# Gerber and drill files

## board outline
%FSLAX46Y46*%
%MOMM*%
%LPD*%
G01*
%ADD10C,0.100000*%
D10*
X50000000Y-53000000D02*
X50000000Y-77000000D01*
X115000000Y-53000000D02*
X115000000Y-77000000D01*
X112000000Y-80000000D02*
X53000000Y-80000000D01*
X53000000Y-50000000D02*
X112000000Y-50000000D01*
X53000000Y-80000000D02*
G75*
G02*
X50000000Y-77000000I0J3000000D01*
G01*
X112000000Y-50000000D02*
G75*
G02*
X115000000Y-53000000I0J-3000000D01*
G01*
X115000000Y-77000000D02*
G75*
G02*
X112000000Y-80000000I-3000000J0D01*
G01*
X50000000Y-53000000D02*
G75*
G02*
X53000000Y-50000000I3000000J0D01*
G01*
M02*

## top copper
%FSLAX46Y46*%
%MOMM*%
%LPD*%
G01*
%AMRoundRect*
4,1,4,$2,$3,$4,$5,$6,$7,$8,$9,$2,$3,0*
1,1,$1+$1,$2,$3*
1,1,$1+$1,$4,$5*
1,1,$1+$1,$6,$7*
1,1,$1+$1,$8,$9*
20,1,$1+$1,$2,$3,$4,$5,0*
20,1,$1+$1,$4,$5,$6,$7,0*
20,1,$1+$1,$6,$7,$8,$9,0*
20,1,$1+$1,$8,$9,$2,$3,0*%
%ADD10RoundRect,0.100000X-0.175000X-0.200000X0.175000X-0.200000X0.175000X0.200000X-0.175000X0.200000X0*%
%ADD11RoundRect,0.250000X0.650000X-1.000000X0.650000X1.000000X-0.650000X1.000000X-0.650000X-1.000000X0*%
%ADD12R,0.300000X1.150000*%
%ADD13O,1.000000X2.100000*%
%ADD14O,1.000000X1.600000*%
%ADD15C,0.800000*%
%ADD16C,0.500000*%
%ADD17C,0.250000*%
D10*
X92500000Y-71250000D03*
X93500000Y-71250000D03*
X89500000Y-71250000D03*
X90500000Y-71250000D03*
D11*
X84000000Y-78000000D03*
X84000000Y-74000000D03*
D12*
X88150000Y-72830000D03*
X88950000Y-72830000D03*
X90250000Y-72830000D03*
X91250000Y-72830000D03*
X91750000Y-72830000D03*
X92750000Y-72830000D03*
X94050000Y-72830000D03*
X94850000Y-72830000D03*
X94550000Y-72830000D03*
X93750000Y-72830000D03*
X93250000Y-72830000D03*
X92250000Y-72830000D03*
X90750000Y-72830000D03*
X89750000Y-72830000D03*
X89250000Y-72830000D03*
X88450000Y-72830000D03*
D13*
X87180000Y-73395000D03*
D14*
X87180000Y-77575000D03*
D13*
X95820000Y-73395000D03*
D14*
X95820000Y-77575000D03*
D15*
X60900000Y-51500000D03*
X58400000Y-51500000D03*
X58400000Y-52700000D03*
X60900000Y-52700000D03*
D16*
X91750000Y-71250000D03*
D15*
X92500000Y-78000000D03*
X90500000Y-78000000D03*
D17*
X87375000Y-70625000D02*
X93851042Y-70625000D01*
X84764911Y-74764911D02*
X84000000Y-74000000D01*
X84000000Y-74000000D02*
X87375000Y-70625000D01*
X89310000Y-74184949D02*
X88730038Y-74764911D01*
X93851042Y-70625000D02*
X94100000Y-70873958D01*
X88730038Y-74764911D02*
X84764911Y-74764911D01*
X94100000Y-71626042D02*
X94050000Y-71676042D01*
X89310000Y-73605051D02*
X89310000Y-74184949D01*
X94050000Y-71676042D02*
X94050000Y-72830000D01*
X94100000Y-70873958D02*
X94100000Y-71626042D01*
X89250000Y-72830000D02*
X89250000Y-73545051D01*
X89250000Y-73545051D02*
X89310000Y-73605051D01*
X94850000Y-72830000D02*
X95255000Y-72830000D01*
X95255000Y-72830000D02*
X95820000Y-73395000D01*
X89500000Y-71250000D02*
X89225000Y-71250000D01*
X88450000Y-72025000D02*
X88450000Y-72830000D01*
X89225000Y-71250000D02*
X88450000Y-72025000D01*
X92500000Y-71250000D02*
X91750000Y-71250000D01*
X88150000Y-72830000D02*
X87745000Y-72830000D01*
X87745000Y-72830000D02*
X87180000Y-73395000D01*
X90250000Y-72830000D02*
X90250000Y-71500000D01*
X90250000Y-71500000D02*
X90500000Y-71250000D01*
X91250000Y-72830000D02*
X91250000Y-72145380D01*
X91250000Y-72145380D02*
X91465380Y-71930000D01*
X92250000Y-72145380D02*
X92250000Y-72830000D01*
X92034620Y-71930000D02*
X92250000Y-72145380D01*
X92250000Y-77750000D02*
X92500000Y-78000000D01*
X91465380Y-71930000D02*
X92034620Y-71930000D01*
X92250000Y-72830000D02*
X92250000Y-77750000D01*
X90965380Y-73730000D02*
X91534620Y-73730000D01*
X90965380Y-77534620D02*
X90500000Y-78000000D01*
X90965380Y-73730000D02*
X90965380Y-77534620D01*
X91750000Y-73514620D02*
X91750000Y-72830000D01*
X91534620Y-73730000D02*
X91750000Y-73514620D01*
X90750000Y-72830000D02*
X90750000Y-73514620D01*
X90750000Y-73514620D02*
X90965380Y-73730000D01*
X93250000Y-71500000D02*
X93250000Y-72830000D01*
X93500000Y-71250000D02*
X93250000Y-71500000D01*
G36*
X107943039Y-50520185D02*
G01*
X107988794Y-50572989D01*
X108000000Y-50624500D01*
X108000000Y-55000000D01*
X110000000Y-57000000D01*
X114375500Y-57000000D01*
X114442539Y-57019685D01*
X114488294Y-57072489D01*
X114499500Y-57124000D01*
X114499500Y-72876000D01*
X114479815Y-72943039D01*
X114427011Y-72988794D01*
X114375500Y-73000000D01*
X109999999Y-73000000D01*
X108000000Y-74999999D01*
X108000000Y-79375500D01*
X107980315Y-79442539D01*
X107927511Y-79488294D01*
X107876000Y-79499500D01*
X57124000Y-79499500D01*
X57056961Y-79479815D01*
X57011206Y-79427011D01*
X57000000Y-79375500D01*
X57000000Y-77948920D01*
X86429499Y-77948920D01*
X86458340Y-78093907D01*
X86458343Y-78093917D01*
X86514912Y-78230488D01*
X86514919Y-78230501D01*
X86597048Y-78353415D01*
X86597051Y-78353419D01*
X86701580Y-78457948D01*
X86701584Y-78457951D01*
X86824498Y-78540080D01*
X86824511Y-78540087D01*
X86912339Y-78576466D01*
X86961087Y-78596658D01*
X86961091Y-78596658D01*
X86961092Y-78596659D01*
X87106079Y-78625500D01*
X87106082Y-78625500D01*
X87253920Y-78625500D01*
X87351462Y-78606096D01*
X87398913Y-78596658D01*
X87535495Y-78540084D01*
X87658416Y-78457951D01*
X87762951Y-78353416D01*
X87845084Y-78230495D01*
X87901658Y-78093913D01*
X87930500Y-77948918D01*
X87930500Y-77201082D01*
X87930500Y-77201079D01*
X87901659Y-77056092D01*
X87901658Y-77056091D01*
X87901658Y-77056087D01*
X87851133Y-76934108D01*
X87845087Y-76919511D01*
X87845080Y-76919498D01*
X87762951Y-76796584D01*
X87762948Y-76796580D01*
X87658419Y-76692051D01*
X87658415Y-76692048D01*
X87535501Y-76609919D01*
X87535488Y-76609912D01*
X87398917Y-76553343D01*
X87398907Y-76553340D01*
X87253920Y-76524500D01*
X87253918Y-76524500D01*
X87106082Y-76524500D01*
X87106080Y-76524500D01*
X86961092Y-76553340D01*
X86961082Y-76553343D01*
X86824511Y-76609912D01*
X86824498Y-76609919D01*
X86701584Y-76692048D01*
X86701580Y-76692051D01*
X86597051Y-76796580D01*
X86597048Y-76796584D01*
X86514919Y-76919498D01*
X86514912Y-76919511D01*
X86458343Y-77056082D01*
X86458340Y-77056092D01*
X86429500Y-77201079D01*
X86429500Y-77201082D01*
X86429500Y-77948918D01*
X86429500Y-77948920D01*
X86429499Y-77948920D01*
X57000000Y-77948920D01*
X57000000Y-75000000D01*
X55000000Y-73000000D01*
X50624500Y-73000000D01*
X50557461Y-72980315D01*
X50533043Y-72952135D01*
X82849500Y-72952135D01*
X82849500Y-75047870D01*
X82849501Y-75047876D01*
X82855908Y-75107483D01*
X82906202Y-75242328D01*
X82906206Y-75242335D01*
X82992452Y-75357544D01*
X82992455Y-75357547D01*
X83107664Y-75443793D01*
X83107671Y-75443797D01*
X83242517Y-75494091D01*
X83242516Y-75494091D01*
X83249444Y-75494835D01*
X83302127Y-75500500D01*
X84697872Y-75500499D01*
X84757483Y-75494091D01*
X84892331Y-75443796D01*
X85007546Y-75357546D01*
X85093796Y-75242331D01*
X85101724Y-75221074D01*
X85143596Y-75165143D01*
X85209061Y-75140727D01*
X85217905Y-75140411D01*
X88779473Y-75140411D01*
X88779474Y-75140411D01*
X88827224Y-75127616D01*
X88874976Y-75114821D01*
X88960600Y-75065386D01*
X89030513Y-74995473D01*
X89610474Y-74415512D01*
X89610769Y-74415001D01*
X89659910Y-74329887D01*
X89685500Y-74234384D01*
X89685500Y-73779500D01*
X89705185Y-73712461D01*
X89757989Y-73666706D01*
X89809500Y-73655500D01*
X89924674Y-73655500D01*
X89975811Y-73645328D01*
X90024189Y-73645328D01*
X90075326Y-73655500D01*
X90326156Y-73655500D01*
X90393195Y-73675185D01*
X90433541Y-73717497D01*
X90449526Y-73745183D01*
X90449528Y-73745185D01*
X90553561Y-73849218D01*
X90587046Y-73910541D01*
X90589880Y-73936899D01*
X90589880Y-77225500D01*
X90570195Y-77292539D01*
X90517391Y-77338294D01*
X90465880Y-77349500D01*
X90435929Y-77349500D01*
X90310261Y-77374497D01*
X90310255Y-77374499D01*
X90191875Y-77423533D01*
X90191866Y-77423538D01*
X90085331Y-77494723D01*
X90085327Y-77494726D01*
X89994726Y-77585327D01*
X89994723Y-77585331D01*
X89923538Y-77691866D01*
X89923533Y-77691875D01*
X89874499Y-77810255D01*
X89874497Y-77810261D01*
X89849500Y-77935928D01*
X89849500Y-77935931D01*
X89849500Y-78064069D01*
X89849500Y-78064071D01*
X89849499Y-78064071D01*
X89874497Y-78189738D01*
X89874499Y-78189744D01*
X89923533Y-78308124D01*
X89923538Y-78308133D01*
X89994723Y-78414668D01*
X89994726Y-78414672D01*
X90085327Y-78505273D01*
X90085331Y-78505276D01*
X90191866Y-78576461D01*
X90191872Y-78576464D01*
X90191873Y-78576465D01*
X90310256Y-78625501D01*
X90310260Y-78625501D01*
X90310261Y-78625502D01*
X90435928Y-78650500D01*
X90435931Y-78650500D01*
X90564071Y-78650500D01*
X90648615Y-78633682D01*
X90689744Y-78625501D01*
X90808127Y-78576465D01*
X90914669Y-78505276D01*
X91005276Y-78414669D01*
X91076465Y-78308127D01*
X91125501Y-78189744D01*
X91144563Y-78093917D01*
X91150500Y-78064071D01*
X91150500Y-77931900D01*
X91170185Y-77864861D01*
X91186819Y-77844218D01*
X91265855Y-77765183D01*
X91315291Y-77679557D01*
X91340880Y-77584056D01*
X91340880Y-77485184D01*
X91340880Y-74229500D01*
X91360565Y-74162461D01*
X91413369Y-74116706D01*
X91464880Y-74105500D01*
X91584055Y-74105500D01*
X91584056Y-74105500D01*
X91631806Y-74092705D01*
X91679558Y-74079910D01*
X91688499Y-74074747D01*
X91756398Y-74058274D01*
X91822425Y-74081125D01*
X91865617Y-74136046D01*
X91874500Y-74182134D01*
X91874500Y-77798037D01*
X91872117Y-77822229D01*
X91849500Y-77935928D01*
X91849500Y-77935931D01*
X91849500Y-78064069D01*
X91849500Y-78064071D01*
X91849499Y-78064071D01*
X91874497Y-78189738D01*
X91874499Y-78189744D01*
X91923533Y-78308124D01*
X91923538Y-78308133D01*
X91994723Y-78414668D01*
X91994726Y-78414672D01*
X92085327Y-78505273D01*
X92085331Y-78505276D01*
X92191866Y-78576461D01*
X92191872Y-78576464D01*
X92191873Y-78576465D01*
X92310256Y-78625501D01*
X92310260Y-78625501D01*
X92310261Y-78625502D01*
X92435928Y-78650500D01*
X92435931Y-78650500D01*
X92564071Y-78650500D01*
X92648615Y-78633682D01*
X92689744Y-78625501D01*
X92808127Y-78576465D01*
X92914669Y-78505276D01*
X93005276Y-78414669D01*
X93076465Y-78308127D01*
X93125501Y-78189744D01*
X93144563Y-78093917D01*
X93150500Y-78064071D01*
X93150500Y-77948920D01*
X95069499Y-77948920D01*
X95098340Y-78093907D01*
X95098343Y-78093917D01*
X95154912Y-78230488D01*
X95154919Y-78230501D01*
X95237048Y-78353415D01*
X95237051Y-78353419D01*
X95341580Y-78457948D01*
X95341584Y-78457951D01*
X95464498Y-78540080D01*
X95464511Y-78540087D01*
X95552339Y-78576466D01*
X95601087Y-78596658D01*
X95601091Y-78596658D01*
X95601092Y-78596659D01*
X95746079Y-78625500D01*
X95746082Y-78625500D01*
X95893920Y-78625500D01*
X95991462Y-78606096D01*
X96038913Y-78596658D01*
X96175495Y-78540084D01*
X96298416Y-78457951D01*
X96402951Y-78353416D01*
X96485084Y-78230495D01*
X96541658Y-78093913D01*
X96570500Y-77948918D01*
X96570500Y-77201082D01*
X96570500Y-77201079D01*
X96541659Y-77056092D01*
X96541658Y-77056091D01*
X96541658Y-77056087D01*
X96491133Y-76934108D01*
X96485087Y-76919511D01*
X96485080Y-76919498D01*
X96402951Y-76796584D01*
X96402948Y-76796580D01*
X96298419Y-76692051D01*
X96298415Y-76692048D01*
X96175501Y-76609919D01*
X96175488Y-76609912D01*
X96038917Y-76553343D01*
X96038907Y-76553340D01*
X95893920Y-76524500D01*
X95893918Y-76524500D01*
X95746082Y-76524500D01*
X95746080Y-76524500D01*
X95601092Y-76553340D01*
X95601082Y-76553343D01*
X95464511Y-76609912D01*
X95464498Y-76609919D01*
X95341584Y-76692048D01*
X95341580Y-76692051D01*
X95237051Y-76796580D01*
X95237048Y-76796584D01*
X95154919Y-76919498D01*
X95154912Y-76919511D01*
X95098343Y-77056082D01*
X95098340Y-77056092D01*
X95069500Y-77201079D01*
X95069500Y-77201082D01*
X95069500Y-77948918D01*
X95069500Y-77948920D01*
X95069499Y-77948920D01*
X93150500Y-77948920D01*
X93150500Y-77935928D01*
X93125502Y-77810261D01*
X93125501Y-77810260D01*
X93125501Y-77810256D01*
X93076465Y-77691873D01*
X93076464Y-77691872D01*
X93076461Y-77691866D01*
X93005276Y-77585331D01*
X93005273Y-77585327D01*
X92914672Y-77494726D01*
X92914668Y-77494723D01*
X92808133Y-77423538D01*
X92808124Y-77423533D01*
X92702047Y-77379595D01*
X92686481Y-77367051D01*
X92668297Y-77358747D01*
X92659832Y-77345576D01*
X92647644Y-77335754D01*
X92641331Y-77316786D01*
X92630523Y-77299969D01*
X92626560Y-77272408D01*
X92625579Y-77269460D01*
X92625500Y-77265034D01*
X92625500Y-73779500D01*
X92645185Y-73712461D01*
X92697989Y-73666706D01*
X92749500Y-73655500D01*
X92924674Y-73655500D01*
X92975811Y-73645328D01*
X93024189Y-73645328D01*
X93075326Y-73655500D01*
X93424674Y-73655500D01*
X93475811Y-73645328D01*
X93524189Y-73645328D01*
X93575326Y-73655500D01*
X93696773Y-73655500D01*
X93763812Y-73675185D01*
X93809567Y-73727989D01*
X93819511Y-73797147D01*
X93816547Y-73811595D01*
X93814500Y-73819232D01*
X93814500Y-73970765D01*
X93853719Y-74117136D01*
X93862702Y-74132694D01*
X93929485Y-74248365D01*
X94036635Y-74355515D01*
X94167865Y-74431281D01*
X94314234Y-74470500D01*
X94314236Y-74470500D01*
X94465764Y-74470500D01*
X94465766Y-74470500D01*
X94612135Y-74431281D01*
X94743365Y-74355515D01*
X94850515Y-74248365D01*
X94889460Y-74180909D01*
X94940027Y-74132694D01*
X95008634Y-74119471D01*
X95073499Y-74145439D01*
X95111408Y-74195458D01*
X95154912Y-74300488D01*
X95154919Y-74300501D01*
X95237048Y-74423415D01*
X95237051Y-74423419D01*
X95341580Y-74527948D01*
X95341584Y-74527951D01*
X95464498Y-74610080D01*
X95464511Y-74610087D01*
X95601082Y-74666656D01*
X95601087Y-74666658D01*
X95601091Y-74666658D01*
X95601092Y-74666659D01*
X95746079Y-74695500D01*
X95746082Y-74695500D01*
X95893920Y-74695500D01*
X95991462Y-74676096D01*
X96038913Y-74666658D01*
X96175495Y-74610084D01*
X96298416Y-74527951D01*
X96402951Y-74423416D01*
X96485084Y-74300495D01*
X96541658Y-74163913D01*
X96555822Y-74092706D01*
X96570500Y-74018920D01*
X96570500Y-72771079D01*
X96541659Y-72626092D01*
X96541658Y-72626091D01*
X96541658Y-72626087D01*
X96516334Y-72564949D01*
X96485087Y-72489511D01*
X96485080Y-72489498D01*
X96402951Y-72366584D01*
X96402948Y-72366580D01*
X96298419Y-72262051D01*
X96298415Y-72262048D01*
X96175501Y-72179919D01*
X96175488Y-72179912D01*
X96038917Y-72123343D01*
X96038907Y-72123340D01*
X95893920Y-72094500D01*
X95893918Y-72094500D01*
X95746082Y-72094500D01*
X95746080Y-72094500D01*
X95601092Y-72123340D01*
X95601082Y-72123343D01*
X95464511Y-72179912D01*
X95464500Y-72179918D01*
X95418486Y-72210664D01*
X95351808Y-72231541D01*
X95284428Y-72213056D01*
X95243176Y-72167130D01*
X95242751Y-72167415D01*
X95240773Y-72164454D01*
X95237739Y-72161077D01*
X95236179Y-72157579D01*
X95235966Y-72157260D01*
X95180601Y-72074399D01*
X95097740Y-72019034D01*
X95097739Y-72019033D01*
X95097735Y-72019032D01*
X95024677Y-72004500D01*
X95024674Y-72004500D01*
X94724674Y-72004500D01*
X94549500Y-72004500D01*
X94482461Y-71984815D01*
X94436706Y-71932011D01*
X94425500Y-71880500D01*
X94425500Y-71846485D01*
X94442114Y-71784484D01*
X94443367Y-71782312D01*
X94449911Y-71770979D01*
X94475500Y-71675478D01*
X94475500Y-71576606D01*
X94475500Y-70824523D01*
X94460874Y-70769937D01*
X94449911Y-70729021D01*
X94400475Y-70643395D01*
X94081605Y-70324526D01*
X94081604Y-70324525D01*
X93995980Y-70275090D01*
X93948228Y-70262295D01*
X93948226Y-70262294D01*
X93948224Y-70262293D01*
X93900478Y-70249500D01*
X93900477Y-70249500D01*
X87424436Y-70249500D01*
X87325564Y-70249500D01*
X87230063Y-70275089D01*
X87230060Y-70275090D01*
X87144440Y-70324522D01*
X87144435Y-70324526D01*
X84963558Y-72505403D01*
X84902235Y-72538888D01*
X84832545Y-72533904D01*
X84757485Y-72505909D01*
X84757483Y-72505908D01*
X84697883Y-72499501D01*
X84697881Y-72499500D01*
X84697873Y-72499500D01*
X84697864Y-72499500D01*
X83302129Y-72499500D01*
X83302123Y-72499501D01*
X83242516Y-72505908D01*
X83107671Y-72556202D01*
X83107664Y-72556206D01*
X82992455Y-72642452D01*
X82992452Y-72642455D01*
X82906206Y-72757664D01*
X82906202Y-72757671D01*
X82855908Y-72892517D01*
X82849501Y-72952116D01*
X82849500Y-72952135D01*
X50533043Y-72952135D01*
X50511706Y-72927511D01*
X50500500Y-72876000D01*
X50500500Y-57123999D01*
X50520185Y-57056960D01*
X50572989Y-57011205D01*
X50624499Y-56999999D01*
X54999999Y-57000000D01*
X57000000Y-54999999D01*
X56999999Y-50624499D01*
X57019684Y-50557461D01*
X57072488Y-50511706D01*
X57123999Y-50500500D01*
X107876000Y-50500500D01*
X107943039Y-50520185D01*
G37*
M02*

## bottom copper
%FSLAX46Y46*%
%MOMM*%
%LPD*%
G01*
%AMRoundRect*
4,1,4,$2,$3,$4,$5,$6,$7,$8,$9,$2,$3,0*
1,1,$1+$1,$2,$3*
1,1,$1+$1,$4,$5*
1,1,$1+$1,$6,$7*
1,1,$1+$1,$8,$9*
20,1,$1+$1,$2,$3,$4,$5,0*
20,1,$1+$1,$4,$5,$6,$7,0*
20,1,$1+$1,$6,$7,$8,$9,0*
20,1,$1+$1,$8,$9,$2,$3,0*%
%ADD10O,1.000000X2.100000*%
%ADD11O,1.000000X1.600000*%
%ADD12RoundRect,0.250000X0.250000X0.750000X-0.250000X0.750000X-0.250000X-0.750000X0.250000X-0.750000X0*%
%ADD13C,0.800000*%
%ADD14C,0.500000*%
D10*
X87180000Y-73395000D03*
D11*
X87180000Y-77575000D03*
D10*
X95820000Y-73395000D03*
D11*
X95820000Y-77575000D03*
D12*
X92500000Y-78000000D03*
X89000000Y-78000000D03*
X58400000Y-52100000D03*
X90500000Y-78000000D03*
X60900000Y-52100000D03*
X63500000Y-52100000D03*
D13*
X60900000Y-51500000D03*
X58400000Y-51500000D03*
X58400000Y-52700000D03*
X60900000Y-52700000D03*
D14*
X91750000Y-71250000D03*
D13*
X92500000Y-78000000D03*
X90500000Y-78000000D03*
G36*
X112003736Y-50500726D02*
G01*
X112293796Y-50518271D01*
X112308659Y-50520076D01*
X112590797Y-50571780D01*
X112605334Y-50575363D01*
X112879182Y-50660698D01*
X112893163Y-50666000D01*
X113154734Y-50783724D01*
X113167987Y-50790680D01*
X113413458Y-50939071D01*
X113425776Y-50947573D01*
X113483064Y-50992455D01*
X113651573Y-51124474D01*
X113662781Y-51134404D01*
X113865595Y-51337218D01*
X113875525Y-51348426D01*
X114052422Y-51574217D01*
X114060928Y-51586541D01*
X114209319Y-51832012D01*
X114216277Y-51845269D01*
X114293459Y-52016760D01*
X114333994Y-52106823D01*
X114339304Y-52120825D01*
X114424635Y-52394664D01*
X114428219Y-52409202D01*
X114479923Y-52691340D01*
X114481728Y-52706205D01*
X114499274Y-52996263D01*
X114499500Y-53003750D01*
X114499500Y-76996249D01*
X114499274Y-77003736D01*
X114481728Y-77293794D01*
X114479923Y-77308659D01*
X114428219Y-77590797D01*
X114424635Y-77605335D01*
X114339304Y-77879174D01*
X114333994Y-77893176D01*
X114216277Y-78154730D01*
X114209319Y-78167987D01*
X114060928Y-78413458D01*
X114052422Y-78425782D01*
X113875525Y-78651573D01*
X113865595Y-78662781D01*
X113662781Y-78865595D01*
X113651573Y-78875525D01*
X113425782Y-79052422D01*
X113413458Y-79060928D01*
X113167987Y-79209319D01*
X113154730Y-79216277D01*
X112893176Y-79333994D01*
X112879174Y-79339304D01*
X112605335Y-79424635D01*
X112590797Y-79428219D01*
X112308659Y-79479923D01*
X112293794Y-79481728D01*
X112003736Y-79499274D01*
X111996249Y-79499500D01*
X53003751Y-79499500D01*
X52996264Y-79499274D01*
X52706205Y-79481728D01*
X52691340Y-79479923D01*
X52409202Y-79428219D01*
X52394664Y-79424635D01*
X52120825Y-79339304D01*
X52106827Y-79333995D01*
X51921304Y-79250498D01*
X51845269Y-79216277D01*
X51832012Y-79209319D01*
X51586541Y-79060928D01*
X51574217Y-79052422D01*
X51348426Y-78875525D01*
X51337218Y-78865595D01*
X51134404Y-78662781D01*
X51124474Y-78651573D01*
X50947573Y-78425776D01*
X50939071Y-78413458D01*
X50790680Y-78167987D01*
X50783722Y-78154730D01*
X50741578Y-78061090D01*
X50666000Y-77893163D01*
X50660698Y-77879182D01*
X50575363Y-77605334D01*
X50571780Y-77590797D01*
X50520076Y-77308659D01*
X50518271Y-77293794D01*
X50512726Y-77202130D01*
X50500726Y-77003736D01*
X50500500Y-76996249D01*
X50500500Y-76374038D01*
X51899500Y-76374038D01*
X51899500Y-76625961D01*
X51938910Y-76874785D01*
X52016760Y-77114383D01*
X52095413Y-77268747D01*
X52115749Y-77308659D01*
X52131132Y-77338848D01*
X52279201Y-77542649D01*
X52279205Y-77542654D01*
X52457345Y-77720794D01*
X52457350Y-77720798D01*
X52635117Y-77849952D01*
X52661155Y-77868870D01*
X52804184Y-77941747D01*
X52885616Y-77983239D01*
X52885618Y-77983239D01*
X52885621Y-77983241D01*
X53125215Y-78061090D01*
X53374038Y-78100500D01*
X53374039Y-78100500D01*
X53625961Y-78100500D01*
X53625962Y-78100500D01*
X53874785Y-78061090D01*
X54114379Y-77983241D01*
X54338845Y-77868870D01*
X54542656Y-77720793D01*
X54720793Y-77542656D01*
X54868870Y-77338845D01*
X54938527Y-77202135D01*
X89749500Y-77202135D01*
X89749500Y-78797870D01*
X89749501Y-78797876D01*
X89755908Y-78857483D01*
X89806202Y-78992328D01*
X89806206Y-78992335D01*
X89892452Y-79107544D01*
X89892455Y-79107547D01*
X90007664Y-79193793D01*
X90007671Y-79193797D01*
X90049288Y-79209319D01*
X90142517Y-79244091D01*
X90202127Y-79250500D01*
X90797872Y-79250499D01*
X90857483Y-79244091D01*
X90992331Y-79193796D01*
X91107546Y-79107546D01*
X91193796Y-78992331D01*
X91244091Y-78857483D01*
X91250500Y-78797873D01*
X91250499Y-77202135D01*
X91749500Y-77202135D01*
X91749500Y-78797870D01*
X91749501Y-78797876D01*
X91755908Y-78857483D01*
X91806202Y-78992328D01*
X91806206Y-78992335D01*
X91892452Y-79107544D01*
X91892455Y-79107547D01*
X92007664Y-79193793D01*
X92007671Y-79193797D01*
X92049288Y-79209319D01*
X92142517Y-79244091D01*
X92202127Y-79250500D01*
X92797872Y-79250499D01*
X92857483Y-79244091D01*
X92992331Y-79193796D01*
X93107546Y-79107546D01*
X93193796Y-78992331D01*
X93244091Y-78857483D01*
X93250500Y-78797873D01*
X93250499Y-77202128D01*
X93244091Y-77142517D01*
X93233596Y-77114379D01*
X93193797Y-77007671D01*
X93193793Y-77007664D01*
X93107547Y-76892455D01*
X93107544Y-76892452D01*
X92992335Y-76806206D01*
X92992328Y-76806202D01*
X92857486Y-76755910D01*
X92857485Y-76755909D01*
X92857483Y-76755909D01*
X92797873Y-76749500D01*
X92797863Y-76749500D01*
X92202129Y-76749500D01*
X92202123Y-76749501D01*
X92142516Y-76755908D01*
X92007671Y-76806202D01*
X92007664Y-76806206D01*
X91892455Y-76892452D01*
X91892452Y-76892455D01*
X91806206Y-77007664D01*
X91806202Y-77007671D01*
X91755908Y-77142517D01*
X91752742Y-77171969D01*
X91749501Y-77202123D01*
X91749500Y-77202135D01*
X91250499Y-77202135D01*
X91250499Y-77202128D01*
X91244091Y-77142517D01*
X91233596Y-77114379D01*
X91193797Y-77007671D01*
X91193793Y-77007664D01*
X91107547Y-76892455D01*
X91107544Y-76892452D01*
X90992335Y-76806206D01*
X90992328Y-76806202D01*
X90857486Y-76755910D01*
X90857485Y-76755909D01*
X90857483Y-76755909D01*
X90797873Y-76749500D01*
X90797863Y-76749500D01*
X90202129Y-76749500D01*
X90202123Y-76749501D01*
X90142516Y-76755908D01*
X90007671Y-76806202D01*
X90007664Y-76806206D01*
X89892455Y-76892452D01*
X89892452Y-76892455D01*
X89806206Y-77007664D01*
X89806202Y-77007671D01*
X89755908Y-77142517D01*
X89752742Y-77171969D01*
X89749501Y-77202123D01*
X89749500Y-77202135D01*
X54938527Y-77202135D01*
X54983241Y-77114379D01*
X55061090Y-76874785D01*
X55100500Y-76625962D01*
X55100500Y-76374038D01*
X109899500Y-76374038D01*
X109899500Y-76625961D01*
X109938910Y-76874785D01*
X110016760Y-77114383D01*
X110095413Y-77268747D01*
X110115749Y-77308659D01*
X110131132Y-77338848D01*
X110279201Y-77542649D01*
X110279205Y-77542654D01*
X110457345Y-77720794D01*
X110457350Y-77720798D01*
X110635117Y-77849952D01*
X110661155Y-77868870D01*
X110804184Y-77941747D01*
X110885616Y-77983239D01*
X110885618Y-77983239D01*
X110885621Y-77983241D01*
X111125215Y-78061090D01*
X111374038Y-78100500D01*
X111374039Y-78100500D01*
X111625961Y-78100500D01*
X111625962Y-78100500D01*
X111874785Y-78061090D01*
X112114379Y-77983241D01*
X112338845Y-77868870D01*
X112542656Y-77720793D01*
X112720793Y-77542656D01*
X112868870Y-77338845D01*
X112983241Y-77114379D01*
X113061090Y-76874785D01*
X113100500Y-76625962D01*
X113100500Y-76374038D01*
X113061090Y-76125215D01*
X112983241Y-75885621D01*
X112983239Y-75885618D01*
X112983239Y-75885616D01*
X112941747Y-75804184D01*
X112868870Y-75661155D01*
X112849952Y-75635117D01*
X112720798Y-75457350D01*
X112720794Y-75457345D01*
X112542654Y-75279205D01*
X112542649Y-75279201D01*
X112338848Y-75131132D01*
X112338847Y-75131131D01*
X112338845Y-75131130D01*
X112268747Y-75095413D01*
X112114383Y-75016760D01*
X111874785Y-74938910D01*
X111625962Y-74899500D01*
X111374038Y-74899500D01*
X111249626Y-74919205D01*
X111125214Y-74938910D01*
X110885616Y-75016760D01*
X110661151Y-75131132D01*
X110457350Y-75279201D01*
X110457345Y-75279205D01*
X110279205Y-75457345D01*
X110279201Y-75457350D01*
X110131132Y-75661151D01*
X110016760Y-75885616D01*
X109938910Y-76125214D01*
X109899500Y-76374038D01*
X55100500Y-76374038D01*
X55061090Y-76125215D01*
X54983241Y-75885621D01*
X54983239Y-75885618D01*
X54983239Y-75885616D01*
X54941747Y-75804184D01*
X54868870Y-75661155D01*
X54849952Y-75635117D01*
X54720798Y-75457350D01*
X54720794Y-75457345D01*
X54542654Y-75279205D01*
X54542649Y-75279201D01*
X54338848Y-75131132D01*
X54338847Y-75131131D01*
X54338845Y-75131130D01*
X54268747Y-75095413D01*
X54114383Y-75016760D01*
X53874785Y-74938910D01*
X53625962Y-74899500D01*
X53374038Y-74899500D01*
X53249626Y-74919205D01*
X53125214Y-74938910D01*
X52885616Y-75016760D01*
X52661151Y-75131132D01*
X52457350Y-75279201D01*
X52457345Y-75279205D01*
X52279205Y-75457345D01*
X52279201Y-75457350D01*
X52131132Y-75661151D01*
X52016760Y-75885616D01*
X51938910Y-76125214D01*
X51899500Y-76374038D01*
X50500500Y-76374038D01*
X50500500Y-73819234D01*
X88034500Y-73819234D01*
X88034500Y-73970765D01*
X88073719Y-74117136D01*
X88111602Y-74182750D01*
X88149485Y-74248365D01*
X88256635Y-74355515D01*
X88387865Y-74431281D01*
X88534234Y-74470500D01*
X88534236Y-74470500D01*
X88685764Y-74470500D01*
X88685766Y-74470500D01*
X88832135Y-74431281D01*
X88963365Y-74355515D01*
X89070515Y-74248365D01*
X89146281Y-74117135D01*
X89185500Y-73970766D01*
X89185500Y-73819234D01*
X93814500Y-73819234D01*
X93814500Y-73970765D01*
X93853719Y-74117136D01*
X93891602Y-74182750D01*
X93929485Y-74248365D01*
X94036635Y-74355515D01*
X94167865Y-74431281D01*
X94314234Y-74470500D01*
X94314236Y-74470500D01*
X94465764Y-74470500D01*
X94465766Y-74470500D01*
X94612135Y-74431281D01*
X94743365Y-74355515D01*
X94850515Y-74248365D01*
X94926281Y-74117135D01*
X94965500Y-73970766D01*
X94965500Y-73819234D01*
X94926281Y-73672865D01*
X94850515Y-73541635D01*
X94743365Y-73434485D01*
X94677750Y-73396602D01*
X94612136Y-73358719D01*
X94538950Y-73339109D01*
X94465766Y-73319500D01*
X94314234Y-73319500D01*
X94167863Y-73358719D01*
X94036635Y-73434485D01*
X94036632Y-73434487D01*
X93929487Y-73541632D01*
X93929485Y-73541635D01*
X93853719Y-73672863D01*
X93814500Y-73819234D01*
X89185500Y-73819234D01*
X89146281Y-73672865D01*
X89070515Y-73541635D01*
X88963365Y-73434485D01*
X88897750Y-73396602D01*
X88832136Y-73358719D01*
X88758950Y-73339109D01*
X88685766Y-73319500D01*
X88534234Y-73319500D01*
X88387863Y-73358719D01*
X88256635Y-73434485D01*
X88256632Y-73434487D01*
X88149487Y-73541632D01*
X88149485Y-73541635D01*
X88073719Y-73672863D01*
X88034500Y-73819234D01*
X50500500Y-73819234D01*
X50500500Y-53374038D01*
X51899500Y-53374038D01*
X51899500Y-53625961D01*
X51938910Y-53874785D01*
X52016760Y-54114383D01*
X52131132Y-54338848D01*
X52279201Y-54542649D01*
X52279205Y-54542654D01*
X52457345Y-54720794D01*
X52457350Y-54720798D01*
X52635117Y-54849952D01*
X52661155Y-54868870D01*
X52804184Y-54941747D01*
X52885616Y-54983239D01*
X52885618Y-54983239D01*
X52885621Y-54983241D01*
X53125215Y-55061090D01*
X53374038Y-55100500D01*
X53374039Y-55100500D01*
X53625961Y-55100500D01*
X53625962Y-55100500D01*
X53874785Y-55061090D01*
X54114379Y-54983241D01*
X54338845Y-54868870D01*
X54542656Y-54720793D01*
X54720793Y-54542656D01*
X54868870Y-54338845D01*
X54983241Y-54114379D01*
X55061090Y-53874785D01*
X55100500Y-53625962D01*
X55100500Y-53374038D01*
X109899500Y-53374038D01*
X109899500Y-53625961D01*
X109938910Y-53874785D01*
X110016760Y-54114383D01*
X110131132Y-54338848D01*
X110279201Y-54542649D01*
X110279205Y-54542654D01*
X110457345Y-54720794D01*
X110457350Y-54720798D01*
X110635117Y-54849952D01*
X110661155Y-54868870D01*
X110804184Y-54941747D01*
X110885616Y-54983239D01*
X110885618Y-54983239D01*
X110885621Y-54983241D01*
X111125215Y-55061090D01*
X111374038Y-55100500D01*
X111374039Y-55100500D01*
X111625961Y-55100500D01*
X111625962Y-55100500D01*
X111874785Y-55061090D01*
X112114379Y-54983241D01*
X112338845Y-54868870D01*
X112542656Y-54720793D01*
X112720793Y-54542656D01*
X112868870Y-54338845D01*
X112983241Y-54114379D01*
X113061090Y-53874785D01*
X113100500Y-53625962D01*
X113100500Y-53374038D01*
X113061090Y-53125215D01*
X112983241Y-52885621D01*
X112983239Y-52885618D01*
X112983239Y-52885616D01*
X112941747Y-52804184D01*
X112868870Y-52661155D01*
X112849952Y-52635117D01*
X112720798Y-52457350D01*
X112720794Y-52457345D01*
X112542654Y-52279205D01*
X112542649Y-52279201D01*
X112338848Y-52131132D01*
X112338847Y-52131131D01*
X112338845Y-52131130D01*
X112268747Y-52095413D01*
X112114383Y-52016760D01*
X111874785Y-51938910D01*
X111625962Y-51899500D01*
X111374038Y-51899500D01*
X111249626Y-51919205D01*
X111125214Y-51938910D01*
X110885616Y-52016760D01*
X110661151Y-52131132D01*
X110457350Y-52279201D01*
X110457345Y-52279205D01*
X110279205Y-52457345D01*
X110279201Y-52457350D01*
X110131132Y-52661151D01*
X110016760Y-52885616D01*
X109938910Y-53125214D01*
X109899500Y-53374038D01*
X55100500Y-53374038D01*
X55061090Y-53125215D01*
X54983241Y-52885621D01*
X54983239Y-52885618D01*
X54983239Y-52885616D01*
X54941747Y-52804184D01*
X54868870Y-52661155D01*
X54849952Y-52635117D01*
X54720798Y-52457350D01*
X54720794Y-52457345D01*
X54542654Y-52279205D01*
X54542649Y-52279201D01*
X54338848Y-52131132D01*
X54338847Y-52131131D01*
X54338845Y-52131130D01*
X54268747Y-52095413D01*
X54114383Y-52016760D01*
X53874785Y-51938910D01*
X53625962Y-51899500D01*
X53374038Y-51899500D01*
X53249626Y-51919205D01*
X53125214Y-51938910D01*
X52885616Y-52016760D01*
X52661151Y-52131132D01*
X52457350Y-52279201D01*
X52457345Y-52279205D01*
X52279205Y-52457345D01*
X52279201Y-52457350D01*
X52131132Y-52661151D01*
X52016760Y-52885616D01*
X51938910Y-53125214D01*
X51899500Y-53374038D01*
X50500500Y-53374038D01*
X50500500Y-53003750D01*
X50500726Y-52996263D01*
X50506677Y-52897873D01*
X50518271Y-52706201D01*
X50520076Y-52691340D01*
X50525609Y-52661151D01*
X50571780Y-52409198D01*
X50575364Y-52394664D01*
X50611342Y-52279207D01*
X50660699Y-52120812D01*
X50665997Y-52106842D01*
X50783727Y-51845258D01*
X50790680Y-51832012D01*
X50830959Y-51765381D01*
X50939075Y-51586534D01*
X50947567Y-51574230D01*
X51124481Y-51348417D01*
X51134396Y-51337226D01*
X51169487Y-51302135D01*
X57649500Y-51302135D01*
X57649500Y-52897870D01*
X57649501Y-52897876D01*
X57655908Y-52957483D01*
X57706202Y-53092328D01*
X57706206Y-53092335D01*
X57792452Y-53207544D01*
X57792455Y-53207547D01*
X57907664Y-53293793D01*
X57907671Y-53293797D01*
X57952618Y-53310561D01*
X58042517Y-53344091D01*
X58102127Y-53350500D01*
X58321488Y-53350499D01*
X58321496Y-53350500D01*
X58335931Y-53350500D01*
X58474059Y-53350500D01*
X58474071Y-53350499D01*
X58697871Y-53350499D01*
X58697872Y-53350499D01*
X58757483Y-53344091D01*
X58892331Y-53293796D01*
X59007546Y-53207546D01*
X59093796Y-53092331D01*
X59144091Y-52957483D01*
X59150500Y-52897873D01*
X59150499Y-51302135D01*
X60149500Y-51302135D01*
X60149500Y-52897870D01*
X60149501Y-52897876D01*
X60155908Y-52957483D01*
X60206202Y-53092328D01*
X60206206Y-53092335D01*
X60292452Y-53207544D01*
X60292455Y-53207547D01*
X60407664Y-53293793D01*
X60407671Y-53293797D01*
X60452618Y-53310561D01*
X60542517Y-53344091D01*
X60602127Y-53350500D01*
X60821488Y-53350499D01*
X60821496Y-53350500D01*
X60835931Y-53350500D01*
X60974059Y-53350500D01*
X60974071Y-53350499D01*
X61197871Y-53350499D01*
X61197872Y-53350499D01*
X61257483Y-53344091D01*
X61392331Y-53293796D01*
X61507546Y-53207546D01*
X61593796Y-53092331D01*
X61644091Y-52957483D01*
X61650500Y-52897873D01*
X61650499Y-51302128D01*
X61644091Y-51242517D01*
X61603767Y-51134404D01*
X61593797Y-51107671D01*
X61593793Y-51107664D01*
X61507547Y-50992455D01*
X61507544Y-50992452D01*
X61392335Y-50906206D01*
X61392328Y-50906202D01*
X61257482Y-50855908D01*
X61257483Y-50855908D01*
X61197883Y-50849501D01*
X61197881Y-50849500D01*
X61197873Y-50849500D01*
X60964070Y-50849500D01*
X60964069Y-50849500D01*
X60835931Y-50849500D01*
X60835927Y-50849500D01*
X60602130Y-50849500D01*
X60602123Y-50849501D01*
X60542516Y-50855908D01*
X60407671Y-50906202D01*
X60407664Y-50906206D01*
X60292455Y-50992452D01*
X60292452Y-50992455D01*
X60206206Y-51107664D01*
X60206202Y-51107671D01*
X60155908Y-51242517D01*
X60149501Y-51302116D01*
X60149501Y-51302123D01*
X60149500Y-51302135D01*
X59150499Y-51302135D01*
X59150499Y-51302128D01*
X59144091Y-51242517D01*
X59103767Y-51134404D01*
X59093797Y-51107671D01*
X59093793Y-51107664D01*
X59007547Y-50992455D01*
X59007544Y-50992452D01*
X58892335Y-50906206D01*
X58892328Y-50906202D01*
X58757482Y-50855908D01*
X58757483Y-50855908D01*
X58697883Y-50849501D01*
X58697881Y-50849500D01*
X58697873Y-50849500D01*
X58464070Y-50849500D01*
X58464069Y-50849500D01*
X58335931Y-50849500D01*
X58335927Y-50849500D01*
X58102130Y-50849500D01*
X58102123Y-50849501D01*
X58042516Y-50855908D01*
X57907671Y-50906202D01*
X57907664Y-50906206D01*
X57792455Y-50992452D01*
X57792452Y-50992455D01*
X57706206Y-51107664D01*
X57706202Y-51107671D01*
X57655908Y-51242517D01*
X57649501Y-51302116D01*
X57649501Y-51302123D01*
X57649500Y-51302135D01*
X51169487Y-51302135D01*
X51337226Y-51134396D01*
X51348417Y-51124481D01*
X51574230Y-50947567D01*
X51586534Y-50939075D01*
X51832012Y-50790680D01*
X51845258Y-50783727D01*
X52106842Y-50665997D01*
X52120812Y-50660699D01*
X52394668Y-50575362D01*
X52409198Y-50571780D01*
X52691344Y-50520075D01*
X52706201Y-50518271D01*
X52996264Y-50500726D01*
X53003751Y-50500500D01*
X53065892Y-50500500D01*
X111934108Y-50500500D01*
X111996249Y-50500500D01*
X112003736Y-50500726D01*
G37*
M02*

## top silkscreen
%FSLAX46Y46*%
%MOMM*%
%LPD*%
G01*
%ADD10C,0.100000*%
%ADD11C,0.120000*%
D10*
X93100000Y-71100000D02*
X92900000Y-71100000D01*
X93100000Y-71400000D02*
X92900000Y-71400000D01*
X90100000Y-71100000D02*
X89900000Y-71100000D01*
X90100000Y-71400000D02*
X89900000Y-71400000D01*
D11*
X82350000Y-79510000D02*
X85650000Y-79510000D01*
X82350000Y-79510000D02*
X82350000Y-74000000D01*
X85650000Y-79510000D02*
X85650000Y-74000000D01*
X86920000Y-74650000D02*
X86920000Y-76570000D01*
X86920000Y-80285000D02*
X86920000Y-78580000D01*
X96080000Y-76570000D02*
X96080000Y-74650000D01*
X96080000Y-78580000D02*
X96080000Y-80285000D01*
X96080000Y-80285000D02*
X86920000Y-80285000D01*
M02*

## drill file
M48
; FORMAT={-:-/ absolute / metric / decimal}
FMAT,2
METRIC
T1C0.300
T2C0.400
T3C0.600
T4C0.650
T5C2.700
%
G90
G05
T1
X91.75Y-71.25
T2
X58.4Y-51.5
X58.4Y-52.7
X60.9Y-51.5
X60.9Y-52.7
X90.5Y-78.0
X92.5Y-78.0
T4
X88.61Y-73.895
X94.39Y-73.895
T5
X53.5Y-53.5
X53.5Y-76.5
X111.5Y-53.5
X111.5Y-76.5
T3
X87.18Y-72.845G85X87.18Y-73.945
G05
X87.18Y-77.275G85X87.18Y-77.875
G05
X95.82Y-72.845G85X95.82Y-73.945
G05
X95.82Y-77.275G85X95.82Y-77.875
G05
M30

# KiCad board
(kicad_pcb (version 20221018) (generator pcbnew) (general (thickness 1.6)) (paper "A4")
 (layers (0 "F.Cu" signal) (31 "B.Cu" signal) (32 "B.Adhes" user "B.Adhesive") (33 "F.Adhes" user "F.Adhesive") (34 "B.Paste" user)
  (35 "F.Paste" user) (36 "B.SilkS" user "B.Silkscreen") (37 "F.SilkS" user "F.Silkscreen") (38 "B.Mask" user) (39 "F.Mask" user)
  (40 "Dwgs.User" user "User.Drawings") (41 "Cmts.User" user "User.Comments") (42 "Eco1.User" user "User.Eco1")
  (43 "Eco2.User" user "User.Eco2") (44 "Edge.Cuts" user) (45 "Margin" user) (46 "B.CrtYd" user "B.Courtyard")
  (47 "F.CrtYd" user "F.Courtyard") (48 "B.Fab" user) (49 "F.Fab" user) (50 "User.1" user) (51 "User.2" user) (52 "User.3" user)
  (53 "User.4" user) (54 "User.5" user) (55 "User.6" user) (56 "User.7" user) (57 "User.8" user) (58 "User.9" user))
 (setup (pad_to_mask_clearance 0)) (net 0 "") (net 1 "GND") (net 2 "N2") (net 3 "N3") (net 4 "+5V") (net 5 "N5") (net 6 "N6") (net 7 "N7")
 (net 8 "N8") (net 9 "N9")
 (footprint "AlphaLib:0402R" (layer "F.Cu") (at 93 71.25)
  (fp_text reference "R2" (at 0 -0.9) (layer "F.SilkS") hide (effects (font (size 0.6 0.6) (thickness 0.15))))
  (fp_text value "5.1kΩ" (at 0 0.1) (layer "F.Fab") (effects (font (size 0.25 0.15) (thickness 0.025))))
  (fp_line (start 0.1 -0.15) (end -0.1 -0.15) (stroke (width 0.1) (type solid)) (layer "F.SilkS"))
  (fp_line (start 0.1 0.15) (end -0.1 0.15) (stroke (width 0.1) (type solid)) (layer "F.SilkS"))
  (pad "1" smd roundrect (at -0.5 0) (size 0.55 0.6) (layers "F.Cu" "F.Paste" "F.Mask") (roundrect_rratio 0.1818181818) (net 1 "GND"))
  (pad "2" smd roundrect (at 0.5 0) (size 0.55 0.6) (layers "F.Cu" "F.Paste" "F.Mask") (roundrect_rratio 0.1818181818) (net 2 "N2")))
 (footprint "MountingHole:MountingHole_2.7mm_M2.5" (layer "F.Cu") (at 111.5 76.5)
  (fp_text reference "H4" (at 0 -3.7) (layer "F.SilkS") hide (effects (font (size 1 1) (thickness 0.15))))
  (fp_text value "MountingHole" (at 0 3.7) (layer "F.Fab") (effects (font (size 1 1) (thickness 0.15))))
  (pad "" np_thru_hole circle (at 0 0) (size 2.7 2.7) (drill 2.7) (layers "*.Cu" "*.Mask")))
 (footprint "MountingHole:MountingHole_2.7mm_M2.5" (layer "F.Cu") (at 53.5 76.5)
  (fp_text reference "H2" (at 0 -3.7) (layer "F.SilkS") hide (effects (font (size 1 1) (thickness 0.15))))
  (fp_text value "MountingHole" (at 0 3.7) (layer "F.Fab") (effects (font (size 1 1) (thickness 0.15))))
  (pad "" np_thru_hole circle (at 0 0) (size 2.7 2.7) (drill 2.7) (layers "*.Cu" "*.Mask")))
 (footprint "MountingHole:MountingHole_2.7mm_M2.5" (layer "F.Cu") (at 111.5 53.5)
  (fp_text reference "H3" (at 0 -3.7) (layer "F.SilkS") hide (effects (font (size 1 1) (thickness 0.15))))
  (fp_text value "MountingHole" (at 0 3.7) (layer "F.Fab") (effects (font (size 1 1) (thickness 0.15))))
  (pad "" np_thru_hole circle (at 0 0) (size 2.7 2.7) (drill 2.7) (layers "*.Cu" "*.Mask")))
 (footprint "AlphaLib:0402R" (layer "F.Cu") (at 90 71.25)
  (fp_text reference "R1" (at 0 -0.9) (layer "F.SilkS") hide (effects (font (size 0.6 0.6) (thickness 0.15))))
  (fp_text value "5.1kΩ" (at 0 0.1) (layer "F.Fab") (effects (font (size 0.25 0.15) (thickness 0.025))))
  (fp_line (start 0.1 -0.15) (end -0.1 -0.15) (stroke (width 0.1) (type solid)) (layer "F.SilkS"))
  (fp_line (start 0.1 0.15) (end -0.1 0.15) (stroke (width 0.1) (type solid)) (layer "F.SilkS"))
  (pad "1" smd roundrect (at -0.5 0) (size 0.55 0.6) (layers "F.Cu" "F.Paste" "F.Mask") (roundrect_rratio 0.1818181818) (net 1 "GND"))
  (pad "2" smd roundrect (at 0.5 0) (size 0.55 0.6) (layers "F.Cu" "F.Paste" "F.Mask") (roundrect_rratio 0.1818181818) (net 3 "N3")))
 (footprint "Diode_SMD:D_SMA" (layer "F.Cu") (at 84 76 90)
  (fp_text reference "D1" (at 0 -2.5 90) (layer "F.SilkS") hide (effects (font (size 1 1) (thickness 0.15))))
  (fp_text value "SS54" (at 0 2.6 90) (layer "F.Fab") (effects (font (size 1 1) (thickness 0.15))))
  (fp_line (start -3.51 -1.65) (end -3.51 1.65) (stroke (width 0.12) (type solid)) (layer "F.SilkS"))
  (fp_line (start -3.51 -1.65) (end 2 -1.65) (stroke (width 0.12) (type solid)) (layer "F.SilkS"))
  (fp_line (start -3.51 1.65) (end 2 1.65) (stroke (width 0.12) (type solid)) (layer "F.SilkS"))
  (pad "1" smd roundrect (at -2 0 90) (size 2.5 1.8) (layers "F.Cu" "F.Paste" "F.Mask") (roundrect_rratio 0.1388888889) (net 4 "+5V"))
  (pad "2" smd roundrect (at 2 0 90) (size 2.5 1.8) (layers "F.Cu" "F.Paste" "F.Mask") (roundrect_rratio 0.1388888889) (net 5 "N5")))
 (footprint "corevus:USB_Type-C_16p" (layer "F.Cu") (at 91.5 76.5)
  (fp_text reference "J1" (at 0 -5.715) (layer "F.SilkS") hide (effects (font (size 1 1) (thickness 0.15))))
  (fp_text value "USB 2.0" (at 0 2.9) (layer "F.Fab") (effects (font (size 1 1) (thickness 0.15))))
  (fp_line (start -4.58 -1.85) (end -4.58 0.07) (stroke (width 0.12) (type solid)) (layer "F.SilkS"))
  (fp_line (start -4.58 3.785) (end -4.58 2.08) (stroke (width 0.12) (type solid)) (layer "F.SilkS"))
  (fp_line (start 4.58 0.07) (end 4.58 -1.85) (stroke (width 0.12) (type solid)) (layer "F.SilkS"))
  (fp_line (start 4.58 2.08) (end 4.58 3.785) (stroke (width 0.12) (type solid)) (layer "F.SilkS"))
  (fp_line (start 4.58 3.785) (end -4.58 3.785) (stroke (width 0.12) (type solid)) (layer "F.SilkS"))
  (pad "" np_thru_hole circle (at -2.89 -2.605) (size 0.65 0.65) (drill 0.65) (layers "*.Cu" "*.Mask"))
  (pad "" np_thru_hole circle (at 2.89 -2.605) (size 0.65 0.65) (drill 0.65) (layers "*.Cu" "*.Mask"))
  (pad "A1" smd rect (at -3.35 -3.67) (size 0.3 1.15) (layers "F.Cu" "F.Paste" "F.Mask") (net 1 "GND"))
  (pad "A4" smd rect (at -2.55 -3.67) (size 0.3 1.15) (layers "F.Cu" "F.Paste" "F.Mask") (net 5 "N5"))
  (pad "A5" smd rect (at -1.25 -3.67) (size 0.3 1.15) (layers "F.Cu" "F.Paste" "F.Mask") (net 3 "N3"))
  (pad "A6" smd rect (at -0.25 -3.67) (size 0.3 1.15) (layers "F.Cu" "F.Paste" "F.Mask") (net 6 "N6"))
  (pad "A7" smd rect (at 0.25 -3.67) (size 0.3 1.15) (layers "F.Cu" "F.Paste" "F.Mask") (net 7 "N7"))
  (pad "A8" smd rect (at 1.25 -3.67) (size 0.3 1.15) (layers "F.Cu" "F.Paste" "F.Mask") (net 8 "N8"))
  (pad "A9" smd rect (at 2.55 -3.67) (size 0.3 1.15) (layers "F.Cu" "F.Paste" "F.Mask") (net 5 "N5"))
  (pad "A12" smd rect (at 3.35 -3.67) (size 0.3 1.15) (layers "F.Cu" "F.Paste" "F.Mask") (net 1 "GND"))
  (pad "B1" smd rect (at 3.05 -3.67) (size 0.3 1.15) (layers "F.Cu" "F.Paste" "F.Mask") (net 1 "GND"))
  (pad "B4" smd rect (at 2.25 -3.67) (size 0.3 1.15) (layers "F.Cu" "F.Paste" "F.Mask") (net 5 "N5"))
  (pad "B5" smd rect (at 1.75 -3.67) (size 0.3 1.15) (layers "F.Cu" "F.Paste" "F.Mask") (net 2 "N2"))
  (pad "B6" smd rect (at 0.75 -3.67) (size 0.3 1.15) (layers "F.Cu" "F.Paste" "F.Mask") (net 6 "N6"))
  (pad "B7" smd rect (at -0.75 -3.67) (size 0.3 1.15) (layers "F.Cu" "F.Paste" "F.Mask") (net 7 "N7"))
  (pad "B8" smd rect (at -1.75 -3.67) (size 0.3 1.15) (layers "F.Cu" "F.Paste" "F.Mask") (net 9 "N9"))
  (pad "B9" smd rect (at -2.25 -3.67) (size 0.3 1.15) (layers "F.Cu" "F.Paste" "F.Mask") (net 5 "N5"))
  (pad "B12" smd rect (at -3.05 -3.67) (size 0.3 1.15) (layers "F.Cu" "F.Paste" "F.Mask") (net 1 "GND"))
  (pad "S1" thru_hole oval (at -4.32 -3.105) (size 1 2.1) (drill oval 0.6 1.7) (layers "*.Cu" "*.Mask") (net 1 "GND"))
  (pad "S1" thru_hole oval (at -4.32 1.075) (size 1 1.6) (drill oval 0.6 1.2) (layers "*.Cu" "*.Mask") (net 1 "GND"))
  (pad "S1" thru_hole oval (at 4.32 -3.105) (size 1 2.1) (drill oval 0.6 1.7) (layers "*.Cu" "*.Mask") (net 1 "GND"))
  (pad "S1" thru_hole oval (at 4.32 1.075) (size 1 1.6) (drill oval 0.6 1.2) (layers "*.Cu" "*.Mask") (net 1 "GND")))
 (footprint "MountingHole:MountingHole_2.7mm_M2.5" (layer "F.Cu") (at 53.5 53.5)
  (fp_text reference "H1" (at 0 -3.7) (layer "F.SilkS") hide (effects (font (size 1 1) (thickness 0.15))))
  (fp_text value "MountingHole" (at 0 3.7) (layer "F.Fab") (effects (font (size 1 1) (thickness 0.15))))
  (pad "" np_thru_hole circle (at 0 0) (size 2.7 2.7) (drill 2.7) (layers "*.Cu" "*.Mask")))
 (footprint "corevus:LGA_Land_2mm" (layer "B.Cu") (at 92.5 78 180)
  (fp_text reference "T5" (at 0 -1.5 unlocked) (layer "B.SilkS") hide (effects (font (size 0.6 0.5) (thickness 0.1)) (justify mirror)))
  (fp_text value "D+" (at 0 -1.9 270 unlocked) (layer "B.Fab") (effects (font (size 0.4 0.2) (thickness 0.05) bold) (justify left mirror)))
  (pad "1" smd roundrect (at 0 0 180) (size 1 2) (layers "B.Cu" "B.Mask") (roundrect_rratio 0.25) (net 6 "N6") (thermal_bridge_angle 45)))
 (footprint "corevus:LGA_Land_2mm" (layer "B.Cu") (at 89 78 180)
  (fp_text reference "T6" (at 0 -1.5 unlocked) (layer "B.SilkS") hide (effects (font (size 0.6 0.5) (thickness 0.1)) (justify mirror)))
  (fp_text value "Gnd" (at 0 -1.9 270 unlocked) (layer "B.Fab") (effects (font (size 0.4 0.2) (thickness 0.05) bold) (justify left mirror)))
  (pad "1" smd roundrect (at 0 0 180) (size 1 2) (layers "B.Cu" "B.Mask") (roundrect_rratio 0.25) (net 1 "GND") (thermal_bridge_angle 45)))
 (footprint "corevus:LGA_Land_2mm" (layer "B.Cu") (at 58.4 52.1 180)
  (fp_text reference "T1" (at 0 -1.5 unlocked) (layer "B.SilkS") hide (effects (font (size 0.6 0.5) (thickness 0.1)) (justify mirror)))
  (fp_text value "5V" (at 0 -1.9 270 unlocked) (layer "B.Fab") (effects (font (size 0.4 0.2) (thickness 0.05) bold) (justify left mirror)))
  (pad "1" smd roundrect (at 0 0 180) (size 1 2) (layers "B.Cu" "B.Mask") (roundrect_rratio 0.25) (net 4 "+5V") (thermal_bridge_angle 45)))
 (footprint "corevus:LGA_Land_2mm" (layer "B.Cu") (at 90.5 78 180)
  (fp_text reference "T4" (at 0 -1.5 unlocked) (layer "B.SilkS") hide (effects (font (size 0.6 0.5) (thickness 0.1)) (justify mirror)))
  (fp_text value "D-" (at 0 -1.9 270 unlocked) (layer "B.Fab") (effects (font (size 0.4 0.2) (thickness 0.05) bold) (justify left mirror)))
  (pad "1" smd roundrect (at 0 0 180) (size 1 2) (layers "B.Cu" "B.Mask") (roundrect_rratio 0.25) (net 7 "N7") (thermal_bridge_angle 45)))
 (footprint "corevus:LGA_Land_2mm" (layer "B.Cu") (at 60.9 52.1 180)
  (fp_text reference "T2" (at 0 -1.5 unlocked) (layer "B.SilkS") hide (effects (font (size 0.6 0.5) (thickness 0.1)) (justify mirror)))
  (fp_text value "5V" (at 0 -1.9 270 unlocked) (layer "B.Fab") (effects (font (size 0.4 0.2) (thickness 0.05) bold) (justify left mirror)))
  (pad "1" smd roundrect (at 0 0 180) (size 1 2) (layers "B.Cu" "B.Mask") (roundrect_rratio 0.25) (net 4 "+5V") (thermal_bridge_angle 45)))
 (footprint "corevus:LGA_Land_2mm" (layer "B.Cu") (at 63.5 52.1 180)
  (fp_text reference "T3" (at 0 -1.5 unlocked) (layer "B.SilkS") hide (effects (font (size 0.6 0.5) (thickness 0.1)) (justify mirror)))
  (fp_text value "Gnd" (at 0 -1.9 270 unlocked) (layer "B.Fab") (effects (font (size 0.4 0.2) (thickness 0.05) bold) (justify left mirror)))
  (pad "1" smd roundrect (at 0 0 180) (size 1 2) (layers "B.Cu" "B.Mask") (roundrect_rratio 0.25) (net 1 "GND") (thermal_bridge_angle 45)))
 (gr_line (start 50 53) (end 50 77) (stroke (width 0.1) (type default)) (layer "Edge.Cuts"))
 (gr_line (start 115 53) (end 115 77) (stroke (width 0.1) (type default)) (layer "Edge.Cuts"))
 (gr_line (start 112 80) (end 53 80) (stroke (width 0.1) (type default)) (layer "Edge.Cuts"))
 (gr_line (start 53 50) (end 112 50) (stroke (width 0.1) (type default)) (layer "Edge.Cuts"))
 (gr_arc (start 53 80) (mid 50.87868 79.12132) (end 50 77) (stroke (width 0.1) (type default)) (layer "Edge.Cuts"))
 (gr_arc (start 112 50) (mid 114.12132 50.87868) (end 115 53) (stroke (width 0.1) (type default)) (layer "Edge.Cuts"))
 (gr_arc (start 115 77) (mid 114.12132 79.12132) (end 112 80) (stroke (width 0.1) (type default)) (layer "Edge.Cuts"))
 (gr_arc (start 50 53) (mid 50.87868 50.87868) (end 53 50) (stroke (width 0.1) (type default)) (layer "Edge.Cuts"))
 (via (at 60.9 51.5) (size 0.8) (drill 0.4) (layers "F.Cu" "B.Cu") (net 4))
 (via (at 58.4 51.5) (size 0.8) (drill 0.4) (layers "F.Cu" "B.Cu") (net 4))
 (via (at 58.4 52.7) (size 0.8) (drill 0.4) (layers "F.Cu" "B.Cu") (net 4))
 (via (at 60.9 52.7) (size 0.8) (drill 0.4) (layers "F.Cu" "B.Cu") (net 4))
 (segment (start 87.375 70.625) (end 93.851042 70.625) (width 0.25) (layer "F.Cu") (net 5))
 (segment (start 84.764911 74.764911) (end 84 74) (width 0.25) (layer "F.Cu") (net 5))
 (segment (start 84 74) (end 87.375 70.625) (width 0.25) (layer "F.Cu") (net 5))
 (segment (start 89.31 74.184949) (end 88.730038 74.764911) (width 0.25) (layer "F.Cu") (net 5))
 (segment (start 93.851042 70.625) (end 94.1 70.873958) (width 0.25) (layer "F.Cu") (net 5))
 (segment (start 88.730038 74.764911) (end 84.764911 74.764911) (width 0.25) (layer "F.Cu") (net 5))
 (segment (start 94.1 71.626042) (end 94.05 71.676042) (width 0.25) (layer "F.Cu") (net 5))
 (segment (start 89.31 73.605051) (end 89.31 74.184949) (width 0.25) (layer "F.Cu") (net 5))
 (segment (start 94.05 71.676042) (end 94.05 72.83) (width 0.25) (layer "F.Cu") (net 5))
 (segment (start 94.1 70.873958) (end 94.1 71.626042) (width 0.25) (layer "F.Cu") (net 5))
 (segment (start 89.25 72.83) (end 89.25 73.545051) (width 0.25) (layer "F.Cu") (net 5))
 (segment (start 89.25 73.545051) (end 89.31 73.605051) (width 0.25) (layer "F.Cu") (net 5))
 (segment (start 94.85 72.83) (end 95.255 72.83) (width 0.25) (layer "F.Cu") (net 1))
 (segment (start 95.255 72.83) (end 95.82 73.395) (width 0.25) (layer "F.Cu") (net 1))
 (segment (start 89.5 71.25) (end 89.225 71.25) (width 0.25) (layer "F.Cu") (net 1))
 (segment (start 88.45 72.025) (end 88.45 72.83) (width 0.25) (layer "F.Cu") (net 1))
 (segment (start 89.225 71.25) (end 88.45 72.025) (width 0.25) (layer "F.Cu") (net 1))
 (segment (start 92.5 71.25) (end 91.75 71.25) (width 0.25) (layer "F.Cu") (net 1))
 (segment (start 88.15 72.83) (end 87.745 72.83) (width 0.25) (layer "F.Cu") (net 1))
 (segment (start 87.745 72.83) (end 87.18 73.395) (width 0.25) (layer "F.Cu") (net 1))
 (via (at 91.75 71.25) (size 0.5) (drill 0.3) (layers "F.Cu" "B.Cu") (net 1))
 (segment (start 90.25 72.83) (end 90.25 71.5) (width 0.25) (layer "F.Cu") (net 3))
 (segment (start 90.25 71.5) (end 90.5 71.25) (width 0.25) (layer "F.Cu") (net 3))
 (segment (start 91.25 72.83) (end 91.25 72.14538) (width 0.25) (layer "F.Cu") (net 6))
 (segment (start 91.25 72.14538) (end 91.46538 71.93) (width 0.25) (layer "F.Cu") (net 6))
 (segment (start 92.25 72.14538) (end 92.25 72.83) (width 0.25) (layer "F.Cu") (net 6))
 (segment (start 92.03462 71.93) (end 92.25 72.14538) (width 0.25) (layer "F.Cu") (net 6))
 (segment (start 92.25 77.75) (end 92.5 78) (width 0.25) (layer "F.Cu") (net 6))
 (segment (start 91.46538 71.93) (end 92.03462 71.93) (width 0.25) (layer "F.Cu") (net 6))
 (segment (start 92.25 72.83) (end 92.25 77.75) (width 0.25) (layer "F.Cu") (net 6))
 (via (at 92.5 78) (size 0.8) (drill 0.4) (layers "F.Cu" "B.Cu") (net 6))
 (segment (start 90.96538 73.73) (end 91.53462 73.73) (width 0.25) (layer "F.Cu") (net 7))
 (segment (start 90.96538 77.53462) (end 90.5 78) (width 0.25) (layer "F.Cu") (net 7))
 (segment (start 90.96538 73.73) (end 90.96538 77.53462) (width 0.25) (layer "F.Cu") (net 7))
 (segment (start 91.75 73.51462) (end 91.75 72.83) (width 0.25) (layer "F.Cu") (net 7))
 (segment (start 91.53462 73.73) (end 91.75 73.51462) (width 0.25) (layer "F.Cu") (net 7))
 (segment (start 90.75 72.83) (end 90.75 73.51462) (width 0.25) (layer "F.Cu") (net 7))
 (segment (start 90.75 73.51462) (end 90.96538 73.73) (width 0.25) (layer "F.Cu") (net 7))
 (via (at 90.5 78) (size 0.8) (drill 0.4) (layers "F.Cu" "B.Cu") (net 7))
 (segment (start 93.25 71.5) (end 93.25 72.83) (width 0.25) (layer "F.Cu") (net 2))
 (segment (start 93.5 71.25) (end 93.25 71.5) (width 0.25) (layer "F.Cu") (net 2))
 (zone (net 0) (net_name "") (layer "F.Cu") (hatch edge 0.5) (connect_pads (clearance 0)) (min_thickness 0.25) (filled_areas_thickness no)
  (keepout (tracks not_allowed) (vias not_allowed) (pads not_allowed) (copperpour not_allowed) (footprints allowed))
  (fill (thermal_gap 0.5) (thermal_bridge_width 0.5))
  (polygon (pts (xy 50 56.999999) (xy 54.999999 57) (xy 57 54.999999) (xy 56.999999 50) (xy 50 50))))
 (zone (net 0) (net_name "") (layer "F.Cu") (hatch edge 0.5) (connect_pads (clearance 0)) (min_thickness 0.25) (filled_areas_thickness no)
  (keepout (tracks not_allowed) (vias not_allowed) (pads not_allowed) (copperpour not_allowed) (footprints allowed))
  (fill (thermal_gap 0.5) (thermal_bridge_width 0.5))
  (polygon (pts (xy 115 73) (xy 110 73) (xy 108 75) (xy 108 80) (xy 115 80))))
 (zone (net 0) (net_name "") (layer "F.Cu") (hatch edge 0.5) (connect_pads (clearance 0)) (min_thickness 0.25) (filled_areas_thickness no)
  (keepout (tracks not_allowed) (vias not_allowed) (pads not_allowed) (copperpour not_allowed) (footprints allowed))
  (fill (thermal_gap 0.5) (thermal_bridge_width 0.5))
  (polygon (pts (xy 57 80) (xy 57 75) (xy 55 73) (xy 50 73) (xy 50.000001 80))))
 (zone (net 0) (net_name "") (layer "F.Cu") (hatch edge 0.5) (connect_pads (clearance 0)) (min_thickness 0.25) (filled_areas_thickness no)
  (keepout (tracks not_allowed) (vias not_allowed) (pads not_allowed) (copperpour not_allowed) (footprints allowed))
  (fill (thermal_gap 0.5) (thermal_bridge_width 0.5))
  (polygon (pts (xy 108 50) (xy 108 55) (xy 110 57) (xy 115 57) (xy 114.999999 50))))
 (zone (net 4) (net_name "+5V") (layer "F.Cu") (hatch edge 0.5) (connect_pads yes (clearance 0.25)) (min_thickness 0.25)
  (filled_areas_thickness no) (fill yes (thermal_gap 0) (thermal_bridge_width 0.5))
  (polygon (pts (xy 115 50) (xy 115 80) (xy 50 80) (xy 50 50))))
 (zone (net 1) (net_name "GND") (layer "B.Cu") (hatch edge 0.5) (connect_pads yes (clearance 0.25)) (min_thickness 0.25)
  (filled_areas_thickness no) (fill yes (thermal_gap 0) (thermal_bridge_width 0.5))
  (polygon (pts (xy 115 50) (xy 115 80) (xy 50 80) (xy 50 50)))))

